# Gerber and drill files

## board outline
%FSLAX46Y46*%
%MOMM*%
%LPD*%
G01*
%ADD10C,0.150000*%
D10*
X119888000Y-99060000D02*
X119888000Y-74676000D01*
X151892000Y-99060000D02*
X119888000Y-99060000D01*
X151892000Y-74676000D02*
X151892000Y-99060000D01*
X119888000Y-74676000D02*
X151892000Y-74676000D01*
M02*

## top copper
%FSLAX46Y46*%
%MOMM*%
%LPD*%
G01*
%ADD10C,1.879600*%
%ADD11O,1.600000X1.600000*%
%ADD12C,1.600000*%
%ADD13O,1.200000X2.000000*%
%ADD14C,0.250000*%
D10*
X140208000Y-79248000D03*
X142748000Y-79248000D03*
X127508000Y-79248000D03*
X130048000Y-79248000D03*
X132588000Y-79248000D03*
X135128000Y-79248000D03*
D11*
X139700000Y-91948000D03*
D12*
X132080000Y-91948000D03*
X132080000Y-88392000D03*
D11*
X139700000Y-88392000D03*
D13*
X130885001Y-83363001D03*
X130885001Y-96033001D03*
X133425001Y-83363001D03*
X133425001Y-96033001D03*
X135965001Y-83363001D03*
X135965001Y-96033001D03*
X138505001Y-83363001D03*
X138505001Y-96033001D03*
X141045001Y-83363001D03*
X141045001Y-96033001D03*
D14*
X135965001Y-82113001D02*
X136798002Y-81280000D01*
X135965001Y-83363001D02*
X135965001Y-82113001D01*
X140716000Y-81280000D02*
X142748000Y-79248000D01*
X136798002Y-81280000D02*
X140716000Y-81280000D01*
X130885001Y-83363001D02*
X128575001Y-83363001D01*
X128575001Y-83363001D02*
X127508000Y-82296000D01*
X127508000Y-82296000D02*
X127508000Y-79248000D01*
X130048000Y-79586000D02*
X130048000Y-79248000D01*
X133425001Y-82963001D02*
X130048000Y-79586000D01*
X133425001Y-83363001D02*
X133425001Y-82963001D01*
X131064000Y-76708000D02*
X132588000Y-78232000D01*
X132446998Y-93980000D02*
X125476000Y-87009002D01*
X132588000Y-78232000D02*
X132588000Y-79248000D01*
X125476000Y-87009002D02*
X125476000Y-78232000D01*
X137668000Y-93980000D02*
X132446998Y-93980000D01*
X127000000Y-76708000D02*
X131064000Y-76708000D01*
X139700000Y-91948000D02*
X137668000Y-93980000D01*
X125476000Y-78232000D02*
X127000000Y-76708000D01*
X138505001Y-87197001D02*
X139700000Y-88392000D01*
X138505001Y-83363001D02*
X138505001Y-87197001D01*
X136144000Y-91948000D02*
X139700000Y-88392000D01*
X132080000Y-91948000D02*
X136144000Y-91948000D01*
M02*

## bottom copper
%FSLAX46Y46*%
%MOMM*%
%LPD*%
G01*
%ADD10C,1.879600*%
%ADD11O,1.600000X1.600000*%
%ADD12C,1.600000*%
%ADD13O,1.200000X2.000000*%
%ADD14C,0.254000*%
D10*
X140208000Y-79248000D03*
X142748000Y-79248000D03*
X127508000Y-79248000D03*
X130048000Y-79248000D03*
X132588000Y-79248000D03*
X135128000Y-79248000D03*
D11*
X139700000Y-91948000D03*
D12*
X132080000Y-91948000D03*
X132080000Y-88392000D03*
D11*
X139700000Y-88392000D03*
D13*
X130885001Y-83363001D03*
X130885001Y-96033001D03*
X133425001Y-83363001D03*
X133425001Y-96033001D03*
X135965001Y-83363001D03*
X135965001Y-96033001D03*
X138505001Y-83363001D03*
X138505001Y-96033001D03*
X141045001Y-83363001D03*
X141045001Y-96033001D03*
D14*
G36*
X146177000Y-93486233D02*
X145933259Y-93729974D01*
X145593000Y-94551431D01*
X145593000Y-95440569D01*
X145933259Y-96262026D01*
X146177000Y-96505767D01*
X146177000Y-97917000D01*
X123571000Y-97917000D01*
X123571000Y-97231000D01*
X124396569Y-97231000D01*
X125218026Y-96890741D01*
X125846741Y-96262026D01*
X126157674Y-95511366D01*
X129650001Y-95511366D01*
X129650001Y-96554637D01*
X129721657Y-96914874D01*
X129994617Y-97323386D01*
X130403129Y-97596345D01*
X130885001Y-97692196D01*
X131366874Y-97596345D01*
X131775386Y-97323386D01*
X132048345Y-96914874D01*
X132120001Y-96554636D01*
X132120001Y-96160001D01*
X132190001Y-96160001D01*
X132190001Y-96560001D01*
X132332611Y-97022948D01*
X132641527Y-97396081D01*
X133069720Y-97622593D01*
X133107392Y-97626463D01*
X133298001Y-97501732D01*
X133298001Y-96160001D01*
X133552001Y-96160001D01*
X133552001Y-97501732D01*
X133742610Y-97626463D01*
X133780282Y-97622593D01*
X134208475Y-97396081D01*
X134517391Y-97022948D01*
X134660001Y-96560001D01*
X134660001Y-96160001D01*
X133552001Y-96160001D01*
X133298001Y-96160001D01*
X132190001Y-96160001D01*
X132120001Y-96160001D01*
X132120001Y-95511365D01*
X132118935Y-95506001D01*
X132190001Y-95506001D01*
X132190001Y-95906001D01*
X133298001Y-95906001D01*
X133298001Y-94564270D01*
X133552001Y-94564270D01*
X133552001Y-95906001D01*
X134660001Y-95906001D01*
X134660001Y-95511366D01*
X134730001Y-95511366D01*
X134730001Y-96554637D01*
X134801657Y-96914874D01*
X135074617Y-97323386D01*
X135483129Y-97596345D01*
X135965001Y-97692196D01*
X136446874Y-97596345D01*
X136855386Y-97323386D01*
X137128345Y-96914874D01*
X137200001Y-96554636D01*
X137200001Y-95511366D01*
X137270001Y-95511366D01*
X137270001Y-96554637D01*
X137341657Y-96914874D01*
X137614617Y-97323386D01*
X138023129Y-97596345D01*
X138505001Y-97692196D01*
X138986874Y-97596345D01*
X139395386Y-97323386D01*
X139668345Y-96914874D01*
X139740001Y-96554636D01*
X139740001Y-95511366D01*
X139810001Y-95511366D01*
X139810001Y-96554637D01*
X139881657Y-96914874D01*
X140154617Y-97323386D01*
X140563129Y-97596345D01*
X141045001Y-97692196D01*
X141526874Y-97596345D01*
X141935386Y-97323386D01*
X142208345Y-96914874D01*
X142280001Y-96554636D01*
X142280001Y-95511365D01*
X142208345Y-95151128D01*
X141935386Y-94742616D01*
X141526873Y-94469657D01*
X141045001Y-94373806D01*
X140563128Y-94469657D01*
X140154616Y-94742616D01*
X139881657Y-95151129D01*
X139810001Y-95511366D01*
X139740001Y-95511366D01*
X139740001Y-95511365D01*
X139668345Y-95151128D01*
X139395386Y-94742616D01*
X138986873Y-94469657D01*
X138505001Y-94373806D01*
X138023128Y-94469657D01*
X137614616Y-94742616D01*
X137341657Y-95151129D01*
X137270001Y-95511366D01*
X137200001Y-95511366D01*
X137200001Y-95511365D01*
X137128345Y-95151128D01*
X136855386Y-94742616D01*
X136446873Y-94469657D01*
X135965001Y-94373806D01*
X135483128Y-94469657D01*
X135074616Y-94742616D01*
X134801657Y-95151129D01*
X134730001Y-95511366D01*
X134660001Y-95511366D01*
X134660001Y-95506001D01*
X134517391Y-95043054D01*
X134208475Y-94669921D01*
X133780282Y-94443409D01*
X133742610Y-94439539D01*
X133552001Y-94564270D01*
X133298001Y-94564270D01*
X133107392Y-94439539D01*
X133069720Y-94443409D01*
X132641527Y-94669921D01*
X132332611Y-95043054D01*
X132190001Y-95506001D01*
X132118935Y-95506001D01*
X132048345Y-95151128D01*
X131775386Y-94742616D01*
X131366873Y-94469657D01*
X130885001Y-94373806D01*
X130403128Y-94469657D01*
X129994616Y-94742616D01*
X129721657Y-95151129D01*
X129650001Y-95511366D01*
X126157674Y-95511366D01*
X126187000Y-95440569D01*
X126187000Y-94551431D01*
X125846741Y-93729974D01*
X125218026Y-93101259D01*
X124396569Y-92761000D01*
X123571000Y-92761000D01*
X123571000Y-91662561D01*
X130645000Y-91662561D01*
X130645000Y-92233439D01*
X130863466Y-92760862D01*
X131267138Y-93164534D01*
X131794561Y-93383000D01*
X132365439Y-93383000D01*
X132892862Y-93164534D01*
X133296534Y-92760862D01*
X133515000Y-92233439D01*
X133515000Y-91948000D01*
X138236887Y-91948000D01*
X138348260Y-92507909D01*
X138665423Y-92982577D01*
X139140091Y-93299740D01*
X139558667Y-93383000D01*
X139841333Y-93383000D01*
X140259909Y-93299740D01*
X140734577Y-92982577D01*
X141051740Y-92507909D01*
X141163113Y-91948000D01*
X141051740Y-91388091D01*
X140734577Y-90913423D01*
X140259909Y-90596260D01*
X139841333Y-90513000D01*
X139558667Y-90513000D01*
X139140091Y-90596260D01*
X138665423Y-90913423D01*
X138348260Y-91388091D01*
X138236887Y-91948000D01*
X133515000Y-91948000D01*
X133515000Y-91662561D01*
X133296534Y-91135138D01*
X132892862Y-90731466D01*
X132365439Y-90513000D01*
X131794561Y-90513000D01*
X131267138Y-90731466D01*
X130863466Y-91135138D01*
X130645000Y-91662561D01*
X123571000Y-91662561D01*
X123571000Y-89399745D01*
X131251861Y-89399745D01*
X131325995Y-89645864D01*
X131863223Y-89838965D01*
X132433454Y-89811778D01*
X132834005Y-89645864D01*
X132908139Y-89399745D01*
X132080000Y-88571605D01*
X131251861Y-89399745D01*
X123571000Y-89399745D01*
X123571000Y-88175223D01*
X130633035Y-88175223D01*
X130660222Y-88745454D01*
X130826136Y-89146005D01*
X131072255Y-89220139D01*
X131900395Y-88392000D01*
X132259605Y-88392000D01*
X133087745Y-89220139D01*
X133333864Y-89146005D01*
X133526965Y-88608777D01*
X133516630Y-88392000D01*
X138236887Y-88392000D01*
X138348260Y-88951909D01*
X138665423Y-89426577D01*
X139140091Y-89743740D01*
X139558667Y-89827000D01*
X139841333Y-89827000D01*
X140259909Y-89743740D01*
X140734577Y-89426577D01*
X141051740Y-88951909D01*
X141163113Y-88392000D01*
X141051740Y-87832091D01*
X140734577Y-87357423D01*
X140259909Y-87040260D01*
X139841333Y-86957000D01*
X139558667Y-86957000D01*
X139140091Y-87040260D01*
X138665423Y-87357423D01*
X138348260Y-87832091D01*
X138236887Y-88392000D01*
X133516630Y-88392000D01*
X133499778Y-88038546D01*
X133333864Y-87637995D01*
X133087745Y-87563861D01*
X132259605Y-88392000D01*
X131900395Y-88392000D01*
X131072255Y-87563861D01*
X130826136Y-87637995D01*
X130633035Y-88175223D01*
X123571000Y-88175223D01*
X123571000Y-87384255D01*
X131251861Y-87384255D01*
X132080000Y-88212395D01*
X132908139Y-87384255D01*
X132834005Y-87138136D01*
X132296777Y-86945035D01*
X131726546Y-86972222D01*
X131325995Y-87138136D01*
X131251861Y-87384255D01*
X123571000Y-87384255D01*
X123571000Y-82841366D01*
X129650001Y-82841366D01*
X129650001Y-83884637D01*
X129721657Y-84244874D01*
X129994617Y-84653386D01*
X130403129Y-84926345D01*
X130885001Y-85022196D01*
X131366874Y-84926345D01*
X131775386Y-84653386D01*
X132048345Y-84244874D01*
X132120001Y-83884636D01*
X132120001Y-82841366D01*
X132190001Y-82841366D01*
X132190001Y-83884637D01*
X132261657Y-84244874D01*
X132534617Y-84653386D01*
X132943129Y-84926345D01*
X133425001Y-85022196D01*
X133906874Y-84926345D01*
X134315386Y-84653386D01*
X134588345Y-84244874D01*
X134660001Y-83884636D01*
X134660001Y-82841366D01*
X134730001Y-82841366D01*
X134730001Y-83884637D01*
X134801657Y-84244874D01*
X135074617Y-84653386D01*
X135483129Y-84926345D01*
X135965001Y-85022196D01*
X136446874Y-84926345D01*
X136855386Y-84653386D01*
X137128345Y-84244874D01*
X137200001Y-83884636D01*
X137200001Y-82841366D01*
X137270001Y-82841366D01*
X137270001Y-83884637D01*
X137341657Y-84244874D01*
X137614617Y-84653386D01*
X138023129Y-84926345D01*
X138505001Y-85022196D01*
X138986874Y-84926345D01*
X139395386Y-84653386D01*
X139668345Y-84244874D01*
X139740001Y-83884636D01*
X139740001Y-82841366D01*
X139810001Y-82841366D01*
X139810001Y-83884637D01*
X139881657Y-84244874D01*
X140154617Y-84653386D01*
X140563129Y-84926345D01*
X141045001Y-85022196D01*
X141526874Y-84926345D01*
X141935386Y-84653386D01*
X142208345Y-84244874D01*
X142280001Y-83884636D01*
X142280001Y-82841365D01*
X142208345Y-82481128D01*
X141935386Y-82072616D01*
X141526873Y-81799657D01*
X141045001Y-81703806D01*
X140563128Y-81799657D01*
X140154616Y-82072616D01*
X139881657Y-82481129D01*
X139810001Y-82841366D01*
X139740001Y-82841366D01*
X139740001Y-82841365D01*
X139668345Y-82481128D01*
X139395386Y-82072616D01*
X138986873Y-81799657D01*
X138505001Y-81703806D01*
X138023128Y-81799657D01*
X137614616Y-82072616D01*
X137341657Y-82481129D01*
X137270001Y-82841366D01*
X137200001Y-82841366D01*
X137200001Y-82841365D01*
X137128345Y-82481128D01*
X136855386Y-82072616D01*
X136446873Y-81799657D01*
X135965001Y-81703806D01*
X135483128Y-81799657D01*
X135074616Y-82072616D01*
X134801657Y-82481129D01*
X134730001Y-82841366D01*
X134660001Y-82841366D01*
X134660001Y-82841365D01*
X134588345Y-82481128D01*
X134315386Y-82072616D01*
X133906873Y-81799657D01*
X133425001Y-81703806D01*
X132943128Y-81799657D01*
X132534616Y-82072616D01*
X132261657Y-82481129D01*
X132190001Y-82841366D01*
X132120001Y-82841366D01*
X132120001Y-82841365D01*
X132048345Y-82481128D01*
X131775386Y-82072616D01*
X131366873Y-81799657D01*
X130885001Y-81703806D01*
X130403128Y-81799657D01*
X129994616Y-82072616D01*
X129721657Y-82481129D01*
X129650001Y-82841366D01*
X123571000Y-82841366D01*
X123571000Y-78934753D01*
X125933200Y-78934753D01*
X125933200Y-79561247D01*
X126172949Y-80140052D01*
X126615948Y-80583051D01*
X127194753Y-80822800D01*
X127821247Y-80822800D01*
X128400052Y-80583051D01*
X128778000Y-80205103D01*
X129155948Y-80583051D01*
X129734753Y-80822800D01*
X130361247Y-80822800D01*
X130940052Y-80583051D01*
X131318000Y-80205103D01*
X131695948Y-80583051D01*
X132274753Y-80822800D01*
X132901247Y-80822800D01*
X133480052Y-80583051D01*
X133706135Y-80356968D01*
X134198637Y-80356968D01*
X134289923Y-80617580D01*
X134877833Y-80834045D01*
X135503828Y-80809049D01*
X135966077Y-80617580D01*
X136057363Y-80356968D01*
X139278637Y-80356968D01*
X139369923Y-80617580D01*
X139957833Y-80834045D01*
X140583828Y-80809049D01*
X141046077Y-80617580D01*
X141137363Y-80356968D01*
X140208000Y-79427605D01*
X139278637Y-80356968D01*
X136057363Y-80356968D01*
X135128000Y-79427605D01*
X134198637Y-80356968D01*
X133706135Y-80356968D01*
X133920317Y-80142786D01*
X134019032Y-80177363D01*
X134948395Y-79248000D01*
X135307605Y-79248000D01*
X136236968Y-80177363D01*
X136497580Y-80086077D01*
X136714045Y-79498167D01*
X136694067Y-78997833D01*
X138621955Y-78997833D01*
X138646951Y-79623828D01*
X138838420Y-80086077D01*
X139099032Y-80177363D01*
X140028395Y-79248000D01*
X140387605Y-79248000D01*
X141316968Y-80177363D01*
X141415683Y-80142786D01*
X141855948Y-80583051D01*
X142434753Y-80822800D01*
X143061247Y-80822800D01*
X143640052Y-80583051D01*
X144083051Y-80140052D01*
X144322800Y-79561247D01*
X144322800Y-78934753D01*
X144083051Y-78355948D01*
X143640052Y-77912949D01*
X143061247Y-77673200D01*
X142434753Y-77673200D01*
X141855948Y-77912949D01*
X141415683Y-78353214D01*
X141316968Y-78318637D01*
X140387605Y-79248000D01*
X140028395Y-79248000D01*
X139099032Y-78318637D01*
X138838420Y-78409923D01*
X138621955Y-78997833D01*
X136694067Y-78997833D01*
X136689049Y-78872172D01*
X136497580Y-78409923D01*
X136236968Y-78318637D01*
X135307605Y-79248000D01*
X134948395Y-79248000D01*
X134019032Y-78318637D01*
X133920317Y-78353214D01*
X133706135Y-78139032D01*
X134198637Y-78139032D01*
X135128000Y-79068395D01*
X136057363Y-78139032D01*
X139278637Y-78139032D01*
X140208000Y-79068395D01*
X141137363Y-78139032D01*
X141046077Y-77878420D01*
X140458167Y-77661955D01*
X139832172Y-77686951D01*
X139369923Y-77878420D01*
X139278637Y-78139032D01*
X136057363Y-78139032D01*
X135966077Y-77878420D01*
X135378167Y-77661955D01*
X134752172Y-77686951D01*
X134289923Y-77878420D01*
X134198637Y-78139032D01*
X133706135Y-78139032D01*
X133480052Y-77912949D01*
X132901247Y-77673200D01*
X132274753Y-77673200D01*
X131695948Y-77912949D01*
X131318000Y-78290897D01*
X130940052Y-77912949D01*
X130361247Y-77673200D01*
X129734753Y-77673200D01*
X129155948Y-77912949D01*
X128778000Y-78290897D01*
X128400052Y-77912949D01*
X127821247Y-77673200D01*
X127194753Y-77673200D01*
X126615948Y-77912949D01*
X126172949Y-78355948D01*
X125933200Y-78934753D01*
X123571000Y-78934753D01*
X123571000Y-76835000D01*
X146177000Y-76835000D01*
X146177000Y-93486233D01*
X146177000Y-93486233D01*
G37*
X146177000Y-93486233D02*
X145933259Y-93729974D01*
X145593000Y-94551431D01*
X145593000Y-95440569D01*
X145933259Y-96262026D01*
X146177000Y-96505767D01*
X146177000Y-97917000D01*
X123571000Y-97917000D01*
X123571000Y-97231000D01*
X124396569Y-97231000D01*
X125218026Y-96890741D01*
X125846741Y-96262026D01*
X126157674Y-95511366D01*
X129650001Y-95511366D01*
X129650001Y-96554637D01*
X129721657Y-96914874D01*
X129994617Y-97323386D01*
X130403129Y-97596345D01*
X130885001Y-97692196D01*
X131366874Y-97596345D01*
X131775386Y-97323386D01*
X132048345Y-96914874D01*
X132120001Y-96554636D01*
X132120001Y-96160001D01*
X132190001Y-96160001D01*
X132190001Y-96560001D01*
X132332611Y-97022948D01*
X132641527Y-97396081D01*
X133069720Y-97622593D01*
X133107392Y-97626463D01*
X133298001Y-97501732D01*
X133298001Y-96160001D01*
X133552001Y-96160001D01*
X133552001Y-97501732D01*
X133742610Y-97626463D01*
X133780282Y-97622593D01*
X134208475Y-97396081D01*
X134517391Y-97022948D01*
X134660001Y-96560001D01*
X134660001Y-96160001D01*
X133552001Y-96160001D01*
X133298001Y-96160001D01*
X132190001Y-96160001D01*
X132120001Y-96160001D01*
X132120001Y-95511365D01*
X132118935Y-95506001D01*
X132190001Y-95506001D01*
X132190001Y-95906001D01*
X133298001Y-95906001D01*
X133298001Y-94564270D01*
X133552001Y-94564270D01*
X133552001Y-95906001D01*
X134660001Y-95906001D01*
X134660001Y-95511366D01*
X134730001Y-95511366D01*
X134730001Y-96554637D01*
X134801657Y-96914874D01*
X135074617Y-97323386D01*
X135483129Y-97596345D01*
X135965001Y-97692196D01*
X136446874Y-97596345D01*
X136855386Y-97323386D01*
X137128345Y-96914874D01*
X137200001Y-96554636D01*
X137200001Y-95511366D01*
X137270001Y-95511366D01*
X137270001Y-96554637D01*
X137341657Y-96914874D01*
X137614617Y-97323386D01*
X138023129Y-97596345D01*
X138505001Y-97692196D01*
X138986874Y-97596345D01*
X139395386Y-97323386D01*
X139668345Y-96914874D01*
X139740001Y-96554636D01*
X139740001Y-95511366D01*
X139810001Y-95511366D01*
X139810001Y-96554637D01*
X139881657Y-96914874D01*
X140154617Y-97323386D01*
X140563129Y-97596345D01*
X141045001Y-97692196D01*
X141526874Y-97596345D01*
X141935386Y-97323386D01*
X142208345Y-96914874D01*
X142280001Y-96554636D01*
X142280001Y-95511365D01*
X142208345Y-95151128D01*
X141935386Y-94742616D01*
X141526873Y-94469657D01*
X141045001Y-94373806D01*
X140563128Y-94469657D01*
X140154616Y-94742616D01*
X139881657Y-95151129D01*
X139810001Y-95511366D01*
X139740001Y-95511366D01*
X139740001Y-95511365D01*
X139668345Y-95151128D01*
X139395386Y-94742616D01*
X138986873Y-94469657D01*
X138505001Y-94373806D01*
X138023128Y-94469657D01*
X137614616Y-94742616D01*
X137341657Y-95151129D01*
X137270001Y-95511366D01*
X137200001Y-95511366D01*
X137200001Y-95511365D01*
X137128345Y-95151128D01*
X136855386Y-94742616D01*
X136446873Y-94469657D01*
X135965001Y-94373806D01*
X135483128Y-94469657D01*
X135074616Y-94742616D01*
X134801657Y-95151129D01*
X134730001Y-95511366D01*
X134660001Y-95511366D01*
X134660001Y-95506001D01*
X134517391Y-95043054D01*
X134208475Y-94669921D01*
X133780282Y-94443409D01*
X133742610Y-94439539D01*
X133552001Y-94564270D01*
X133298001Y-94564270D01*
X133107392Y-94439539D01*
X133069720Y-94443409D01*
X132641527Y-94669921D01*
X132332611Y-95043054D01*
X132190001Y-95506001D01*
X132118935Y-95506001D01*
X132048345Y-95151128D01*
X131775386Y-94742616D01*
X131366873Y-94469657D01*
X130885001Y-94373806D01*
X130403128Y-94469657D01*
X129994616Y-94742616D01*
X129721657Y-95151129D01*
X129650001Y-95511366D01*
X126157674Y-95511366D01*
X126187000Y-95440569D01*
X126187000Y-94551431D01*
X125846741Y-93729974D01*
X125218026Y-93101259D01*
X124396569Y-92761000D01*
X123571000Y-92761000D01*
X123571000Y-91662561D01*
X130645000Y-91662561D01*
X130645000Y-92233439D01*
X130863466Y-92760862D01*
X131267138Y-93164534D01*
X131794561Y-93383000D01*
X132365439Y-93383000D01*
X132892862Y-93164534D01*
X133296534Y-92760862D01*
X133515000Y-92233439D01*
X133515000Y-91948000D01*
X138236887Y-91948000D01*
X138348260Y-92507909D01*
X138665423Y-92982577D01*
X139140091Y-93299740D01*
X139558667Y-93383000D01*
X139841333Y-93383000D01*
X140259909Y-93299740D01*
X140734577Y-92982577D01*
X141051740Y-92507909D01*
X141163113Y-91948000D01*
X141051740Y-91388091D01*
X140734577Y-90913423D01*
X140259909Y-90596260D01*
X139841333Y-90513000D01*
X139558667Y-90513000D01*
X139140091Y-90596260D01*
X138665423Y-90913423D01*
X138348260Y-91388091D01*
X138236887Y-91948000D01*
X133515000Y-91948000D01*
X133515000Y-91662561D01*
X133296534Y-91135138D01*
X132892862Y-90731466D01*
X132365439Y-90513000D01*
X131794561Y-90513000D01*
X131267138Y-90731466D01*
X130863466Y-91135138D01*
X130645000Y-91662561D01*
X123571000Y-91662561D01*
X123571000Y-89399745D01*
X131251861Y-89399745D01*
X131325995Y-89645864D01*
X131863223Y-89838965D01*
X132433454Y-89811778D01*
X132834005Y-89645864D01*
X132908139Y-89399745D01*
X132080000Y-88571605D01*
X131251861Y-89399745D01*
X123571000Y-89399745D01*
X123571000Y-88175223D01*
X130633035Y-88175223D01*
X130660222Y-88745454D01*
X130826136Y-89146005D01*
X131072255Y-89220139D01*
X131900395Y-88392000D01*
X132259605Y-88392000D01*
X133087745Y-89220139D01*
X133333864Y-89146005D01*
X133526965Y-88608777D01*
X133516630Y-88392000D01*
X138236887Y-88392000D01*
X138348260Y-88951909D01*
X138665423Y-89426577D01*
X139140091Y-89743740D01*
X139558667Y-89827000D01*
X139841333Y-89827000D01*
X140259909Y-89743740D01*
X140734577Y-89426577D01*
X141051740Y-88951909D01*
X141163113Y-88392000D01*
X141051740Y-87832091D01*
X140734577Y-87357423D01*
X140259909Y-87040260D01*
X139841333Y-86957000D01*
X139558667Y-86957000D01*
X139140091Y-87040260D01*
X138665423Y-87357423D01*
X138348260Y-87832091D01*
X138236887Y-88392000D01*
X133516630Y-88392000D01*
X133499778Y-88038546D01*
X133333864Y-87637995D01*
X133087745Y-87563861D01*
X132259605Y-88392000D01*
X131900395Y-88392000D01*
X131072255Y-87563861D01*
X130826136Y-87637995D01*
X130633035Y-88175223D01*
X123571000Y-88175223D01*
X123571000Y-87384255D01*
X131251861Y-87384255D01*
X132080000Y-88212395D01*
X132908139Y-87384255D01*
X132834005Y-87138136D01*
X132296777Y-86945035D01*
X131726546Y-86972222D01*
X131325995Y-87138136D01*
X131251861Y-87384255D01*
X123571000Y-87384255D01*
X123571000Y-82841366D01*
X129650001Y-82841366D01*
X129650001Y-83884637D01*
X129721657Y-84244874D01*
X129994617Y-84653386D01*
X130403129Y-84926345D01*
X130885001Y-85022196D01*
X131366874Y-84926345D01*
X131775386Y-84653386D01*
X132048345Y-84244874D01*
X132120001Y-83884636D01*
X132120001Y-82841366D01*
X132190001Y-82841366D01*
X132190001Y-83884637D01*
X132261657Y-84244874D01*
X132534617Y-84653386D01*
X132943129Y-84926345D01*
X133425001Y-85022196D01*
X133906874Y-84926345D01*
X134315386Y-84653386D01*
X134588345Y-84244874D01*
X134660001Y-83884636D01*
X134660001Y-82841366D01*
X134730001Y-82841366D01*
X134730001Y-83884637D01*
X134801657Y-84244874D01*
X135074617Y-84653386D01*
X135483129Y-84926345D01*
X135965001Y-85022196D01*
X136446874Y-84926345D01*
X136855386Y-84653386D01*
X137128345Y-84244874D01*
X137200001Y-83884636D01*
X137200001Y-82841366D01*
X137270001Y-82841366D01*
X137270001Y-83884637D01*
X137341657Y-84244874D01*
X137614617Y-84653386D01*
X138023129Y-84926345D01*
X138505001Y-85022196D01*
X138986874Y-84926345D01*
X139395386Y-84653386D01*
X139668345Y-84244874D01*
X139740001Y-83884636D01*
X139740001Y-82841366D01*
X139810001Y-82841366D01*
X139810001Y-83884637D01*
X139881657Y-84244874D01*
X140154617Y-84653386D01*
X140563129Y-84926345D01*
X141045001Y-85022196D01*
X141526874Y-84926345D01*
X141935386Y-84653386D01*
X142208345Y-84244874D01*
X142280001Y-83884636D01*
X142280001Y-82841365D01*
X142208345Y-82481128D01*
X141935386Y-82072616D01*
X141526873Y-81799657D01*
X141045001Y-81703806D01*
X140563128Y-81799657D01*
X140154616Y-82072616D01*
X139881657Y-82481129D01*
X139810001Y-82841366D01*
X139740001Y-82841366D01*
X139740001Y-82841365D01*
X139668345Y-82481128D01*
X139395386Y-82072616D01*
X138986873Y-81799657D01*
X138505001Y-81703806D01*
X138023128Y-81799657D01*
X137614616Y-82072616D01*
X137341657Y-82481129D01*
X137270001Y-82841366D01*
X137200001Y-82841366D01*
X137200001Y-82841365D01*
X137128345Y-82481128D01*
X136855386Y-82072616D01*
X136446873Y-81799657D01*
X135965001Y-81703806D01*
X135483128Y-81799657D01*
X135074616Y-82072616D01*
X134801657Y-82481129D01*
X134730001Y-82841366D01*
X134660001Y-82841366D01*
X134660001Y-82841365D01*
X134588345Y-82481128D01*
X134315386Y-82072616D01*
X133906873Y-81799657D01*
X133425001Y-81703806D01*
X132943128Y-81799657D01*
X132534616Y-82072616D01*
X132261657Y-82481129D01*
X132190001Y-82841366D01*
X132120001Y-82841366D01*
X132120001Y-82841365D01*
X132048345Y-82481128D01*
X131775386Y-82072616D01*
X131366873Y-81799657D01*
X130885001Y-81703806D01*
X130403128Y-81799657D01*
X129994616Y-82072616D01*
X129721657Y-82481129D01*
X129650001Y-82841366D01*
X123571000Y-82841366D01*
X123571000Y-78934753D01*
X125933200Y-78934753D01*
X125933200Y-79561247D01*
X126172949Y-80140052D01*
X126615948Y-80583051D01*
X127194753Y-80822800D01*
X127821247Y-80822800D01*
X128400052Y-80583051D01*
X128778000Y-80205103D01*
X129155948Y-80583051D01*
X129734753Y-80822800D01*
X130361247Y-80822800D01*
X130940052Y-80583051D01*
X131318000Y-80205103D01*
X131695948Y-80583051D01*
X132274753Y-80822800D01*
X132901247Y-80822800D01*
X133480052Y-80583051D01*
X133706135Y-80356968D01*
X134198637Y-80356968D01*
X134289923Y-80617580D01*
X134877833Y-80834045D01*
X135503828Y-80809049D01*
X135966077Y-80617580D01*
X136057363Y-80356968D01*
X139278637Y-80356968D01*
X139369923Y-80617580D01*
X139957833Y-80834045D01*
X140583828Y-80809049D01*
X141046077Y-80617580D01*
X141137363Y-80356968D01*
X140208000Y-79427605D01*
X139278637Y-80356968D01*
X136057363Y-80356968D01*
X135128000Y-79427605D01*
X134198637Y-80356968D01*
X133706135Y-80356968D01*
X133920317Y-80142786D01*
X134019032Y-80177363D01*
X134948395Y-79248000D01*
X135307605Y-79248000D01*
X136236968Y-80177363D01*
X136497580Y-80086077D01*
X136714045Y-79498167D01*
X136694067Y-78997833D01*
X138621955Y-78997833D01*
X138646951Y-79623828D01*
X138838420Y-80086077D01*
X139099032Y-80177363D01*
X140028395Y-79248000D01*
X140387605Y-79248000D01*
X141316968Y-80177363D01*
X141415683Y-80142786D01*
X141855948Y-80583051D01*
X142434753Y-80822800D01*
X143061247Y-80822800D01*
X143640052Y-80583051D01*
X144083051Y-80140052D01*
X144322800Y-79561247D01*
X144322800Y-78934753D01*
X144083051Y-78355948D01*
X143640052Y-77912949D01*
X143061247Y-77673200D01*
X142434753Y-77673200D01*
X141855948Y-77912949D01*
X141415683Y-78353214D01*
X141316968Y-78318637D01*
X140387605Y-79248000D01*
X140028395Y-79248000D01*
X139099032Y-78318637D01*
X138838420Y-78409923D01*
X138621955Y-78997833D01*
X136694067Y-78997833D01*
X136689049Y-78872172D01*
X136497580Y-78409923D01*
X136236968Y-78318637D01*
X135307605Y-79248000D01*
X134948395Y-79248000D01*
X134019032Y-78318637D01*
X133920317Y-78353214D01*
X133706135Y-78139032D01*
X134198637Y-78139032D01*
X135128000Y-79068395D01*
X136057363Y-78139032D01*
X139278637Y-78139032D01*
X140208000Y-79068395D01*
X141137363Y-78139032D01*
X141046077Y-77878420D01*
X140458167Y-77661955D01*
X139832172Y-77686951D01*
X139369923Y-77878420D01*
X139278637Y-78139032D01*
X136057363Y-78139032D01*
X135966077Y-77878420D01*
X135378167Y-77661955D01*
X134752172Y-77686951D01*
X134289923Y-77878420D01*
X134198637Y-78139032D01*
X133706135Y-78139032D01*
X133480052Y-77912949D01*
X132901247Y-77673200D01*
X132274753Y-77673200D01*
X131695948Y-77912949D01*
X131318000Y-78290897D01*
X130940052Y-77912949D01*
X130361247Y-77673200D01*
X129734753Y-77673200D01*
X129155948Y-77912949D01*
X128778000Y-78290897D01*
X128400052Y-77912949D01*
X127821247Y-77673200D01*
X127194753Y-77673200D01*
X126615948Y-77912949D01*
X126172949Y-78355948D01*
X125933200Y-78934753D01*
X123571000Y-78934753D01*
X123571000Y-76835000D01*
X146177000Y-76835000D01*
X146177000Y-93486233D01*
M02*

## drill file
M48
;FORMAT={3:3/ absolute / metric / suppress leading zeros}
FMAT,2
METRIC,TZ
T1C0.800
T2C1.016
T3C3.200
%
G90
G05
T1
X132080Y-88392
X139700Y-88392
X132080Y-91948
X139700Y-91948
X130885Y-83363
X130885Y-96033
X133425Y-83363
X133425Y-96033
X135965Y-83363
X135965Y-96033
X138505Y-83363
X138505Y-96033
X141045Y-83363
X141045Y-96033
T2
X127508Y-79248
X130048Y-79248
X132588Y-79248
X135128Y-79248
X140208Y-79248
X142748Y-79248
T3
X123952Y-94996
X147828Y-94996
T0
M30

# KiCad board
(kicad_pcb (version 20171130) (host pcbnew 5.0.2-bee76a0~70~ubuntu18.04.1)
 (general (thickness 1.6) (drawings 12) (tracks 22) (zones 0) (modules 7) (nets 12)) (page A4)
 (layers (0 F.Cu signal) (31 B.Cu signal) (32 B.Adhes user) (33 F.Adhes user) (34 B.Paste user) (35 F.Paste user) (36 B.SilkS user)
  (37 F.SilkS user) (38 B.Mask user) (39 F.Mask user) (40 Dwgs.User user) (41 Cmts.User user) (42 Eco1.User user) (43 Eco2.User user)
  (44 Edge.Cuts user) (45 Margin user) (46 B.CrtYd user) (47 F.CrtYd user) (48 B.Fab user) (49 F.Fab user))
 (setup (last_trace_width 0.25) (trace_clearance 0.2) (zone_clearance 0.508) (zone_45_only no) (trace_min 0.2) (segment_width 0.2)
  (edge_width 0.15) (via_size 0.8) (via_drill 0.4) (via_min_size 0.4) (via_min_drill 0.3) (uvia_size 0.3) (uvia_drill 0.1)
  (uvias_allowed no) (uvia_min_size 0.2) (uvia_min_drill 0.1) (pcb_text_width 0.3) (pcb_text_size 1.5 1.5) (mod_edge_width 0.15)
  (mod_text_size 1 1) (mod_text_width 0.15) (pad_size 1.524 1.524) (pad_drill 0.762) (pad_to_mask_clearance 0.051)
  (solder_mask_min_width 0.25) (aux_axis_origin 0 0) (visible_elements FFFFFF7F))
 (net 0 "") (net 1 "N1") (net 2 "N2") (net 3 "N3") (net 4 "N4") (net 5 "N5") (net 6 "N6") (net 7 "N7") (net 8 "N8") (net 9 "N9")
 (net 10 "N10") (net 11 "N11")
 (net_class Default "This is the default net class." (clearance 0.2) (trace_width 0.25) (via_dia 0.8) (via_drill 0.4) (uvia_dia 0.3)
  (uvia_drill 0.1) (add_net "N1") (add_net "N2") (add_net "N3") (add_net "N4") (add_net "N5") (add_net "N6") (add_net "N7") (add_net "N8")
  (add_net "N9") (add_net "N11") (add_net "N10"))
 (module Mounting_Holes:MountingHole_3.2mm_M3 (layer F.Cu) (at 147.828 94.996)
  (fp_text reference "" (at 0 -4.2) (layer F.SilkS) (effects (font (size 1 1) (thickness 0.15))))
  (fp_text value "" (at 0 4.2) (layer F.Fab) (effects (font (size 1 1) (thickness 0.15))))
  (pad 1 np_thru_hole circle (at 0 0) (size 3.2 3.2) (drill 3.2) (layers *.Cu *.Mask)))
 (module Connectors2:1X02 (layer F.Cu) (at 140.208 79.248)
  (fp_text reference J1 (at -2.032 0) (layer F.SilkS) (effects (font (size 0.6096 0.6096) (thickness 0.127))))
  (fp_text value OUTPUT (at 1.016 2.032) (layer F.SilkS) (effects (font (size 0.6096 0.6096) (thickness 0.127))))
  (pad 1 thru_hole circle (at 0 0) (size 1.8796 1.8796) (drill 1.016) (layers *.Cu *.Mask) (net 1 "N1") (solder_mask_margin 0.1016))
  (pad 2 thru_hole circle (at 2.54 0) (size 1.8796 1.8796) (drill 1.016) (layers *.Cu *.Mask) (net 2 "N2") (solder_mask_margin 0.1016)))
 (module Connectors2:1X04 (layer F.Cu) (at 127.508 79.248)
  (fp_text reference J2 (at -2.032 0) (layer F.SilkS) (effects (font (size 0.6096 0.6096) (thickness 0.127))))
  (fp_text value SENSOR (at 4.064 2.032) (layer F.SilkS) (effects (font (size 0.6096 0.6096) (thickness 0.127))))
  (pad 1 thru_hole circle (at 0 0) (size 1.8796 1.8796) (drill 1.016) (layers *.Cu *.Mask) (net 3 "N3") (solder_mask_margin 0.1016))
  (pad 2 thru_hole circle (at 2.54 0) (size 1.8796 1.8796) (drill 1.016) (layers *.Cu *.Mask) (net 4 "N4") (solder_mask_margin 0.1016))
  (pad 3 thru_hole circle (at 5.08 0) (size 1.8796 1.8796) (drill 1.016) (layers *.Cu *.Mask) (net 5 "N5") (solder_mask_margin 0.1016))
  (pad 4 thru_hole circle (at 7.62 0) (size 1.8796 1.8796) (drill 1.016) (layers *.Cu *.Mask) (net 1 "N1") (solder_mask_margin 0.1016)))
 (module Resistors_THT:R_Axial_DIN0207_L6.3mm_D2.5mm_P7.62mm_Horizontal (layer F.Cu) (at 132.08 91.948)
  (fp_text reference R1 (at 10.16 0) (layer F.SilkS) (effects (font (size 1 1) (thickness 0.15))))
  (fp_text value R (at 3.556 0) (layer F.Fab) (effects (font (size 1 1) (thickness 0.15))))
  (pad 2 thru_hole oval (at 7.62 0) (size 1.6 1.6) (drill 0.8) (layers *.Cu *.Mask) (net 5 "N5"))
  (pad 1 thru_hole circle (at 0 0) (size 1.6 1.6) (drill 0.8) (layers *.Cu *.Mask) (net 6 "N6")))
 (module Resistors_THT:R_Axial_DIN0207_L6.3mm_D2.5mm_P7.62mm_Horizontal (layer F.Cu) (at 132.08 88.392)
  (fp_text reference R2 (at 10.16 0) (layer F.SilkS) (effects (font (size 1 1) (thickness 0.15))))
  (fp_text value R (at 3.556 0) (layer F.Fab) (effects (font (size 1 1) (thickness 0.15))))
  (pad 1 thru_hole circle (at 0 0) (size 1.6 1.6) (drill 0.8) (layers *.Cu *.Mask) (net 1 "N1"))
  (pad 2 thru_hole oval (at 7.62 0) (size 1.6 1.6) (drill 0.8) (layers *.Cu *.Mask) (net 6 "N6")))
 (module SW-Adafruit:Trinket (layer F.Cu) (at 135.965001 89.698001)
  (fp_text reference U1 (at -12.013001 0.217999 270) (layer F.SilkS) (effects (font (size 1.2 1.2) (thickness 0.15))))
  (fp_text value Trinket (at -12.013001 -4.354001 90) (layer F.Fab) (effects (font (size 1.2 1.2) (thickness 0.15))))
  (pad 10 thru_hole oval (at -5.08 -6.335) (size 1.2 2) (drill 0.8) (layers *.Cu *.Mask) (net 3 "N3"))
  (pad 1 thru_hole oval (at -5.08 6.335) (size 1.2 2) (drill 0.8) (layers *.Cu *.Mask) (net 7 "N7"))
  (pad 9 thru_hole oval (at -2.54 -6.335) (size 1.2 2) (drill 0.8) (layers *.Cu *.Mask) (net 4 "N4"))
  (pad 2 thru_hole oval (at -2.54 6.335) (size 1.2 2) (drill 0.8) (layers *.Cu *.Mask) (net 1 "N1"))
  (pad 8 thru_hole oval (at 0 -6.335) (size 1.2 2) (drill 0.8) (layers *.Cu *.Mask) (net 2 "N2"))
  (pad 3 thru_hole oval (at 0 6.335) (size 1.2 2) (drill 0.8) (layers *.Cu *.Mask) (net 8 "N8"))
  (pad 7 thru_hole oval (at 2.54 -6.335) (size 1.2 2) (drill 0.8) (layers *.Cu *.Mask) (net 6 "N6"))
  (pad 4 thru_hole oval (at 2.54 6.335) (size 1.2 2) (drill 0.8) (layers *.Cu *.Mask) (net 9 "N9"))
  (pad 6 thru_hole oval (at 5.08 -6.335) (size 1.2 2) (drill 0.8) (layers *.Cu *.Mask) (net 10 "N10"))
  (pad 5 thru_hole oval (at 5.08 6.335) (size 1.2 2) (drill 0.8) (layers *.Cu *.Mask) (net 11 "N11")))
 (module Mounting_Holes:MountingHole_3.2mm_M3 (layer F.Cu) (at 123.952 94.996)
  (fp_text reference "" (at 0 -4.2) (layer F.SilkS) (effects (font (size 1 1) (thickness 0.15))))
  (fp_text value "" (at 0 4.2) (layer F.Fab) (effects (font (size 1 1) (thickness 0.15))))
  (pad 1 np_thru_hole circle (at 0 0) (size 3.2 3.2) (drill 3.2) (layers *.Cu *.Mask)))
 (gr_line (start 119.888 99.06) (end 119.888 74.676) (layer Edge.Cuts) (width 0.15))
 (gr_line (start 151.892 99.06) (end 119.888 99.06) (layer Edge.Cuts) (width 0.15))
 (gr_line (start 151.892 74.676) (end 151.892 99.06) (layer Edge.Cuts) (width 0.15))
 (gr_line (start 119.888 74.676) (end 151.892 74.676) (layer Edge.Cuts) (width 0.15))
 (segment (start 135.965001 82.113001) (end 136.798002 81.28) (width 0.25) (layer F.Cu) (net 2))
 (segment (start 135.965001 83.363001) (end 135.965001 82.113001) (width 0.25) (layer F.Cu) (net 2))
 (segment (start 140.716 81.28) (end 142.748 79.248) (width 0.25) (layer F.Cu) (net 2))
 (segment (start 136.798002 81.28) (end 140.716 81.28) (width 0.25) (layer F.Cu) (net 2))
 (segment (start 130.885001 83.363001) (end 128.575001 83.363001) (width 0.25) (layer F.Cu) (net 3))
 (segment (start 128.575001 83.363001) (end 127.508 82.296) (width 0.25) (layer F.Cu) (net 3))
 (segment (start 127.508 82.296) (end 127.508 79.248) (width 0.25) (layer F.Cu) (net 3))
 (segment (start 130.048 79.586) (end 130.048 79.248) (width 0.25) (layer F.Cu) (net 4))
 (segment (start 133.425001 82.963001) (end 130.048 79.586) (width 0.25) (layer F.Cu) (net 4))
 (segment (start 133.425001 83.363001) (end 133.425001 82.963001) (width 0.25) (layer F.Cu) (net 4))
 (segment (start 131.064 76.708) (end 132.588 78.232) (width 0.25) (layer F.Cu) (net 5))
 (segment (start 132.446998 93.98) (end 125.476 87.009002) (width 0.25) (layer F.Cu) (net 5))
 (segment (start 132.588 78.232) (end 132.588 79.248) (width 0.25) (layer F.Cu) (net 5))
 (segment (start 125.476 87.009002) (end 125.476 78.232) (width 0.25) (layer F.Cu) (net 5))
 (segment (start 137.668 93.98) (end 132.446998 93.98) (width 0.25) (layer F.Cu) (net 5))
 (segment (start 127 76.708) (end 131.064 76.708) (width 0.25) (layer F.Cu) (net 5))
 (segment (start 139.7 91.948) (end 137.668 93.98) (width 0.25) (layer F.Cu) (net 5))
 (segment (start 125.476 78.232) (end 127 76.708) (width 0.25) (layer F.Cu) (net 5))
 (segment (start 138.505001 87.197001) (end 139.7 88.392) (width 0.25) (layer F.Cu) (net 6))
 (segment (start 138.505001 83.363001) (end 138.505001 87.197001) (width 0.25) (layer F.Cu) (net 6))
 (segment (start 136.144 91.948) (end 139.7 88.392) (width 0.25) (layer F.Cu) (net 6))
 (segment (start 132.08 91.948) (end 136.144 91.948) (width 0.25) (layer F.Cu) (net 6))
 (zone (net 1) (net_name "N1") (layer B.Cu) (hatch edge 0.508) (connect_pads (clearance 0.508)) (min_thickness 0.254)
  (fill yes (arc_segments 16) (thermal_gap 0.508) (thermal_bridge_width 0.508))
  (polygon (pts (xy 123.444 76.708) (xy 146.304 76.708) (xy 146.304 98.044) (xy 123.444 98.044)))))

